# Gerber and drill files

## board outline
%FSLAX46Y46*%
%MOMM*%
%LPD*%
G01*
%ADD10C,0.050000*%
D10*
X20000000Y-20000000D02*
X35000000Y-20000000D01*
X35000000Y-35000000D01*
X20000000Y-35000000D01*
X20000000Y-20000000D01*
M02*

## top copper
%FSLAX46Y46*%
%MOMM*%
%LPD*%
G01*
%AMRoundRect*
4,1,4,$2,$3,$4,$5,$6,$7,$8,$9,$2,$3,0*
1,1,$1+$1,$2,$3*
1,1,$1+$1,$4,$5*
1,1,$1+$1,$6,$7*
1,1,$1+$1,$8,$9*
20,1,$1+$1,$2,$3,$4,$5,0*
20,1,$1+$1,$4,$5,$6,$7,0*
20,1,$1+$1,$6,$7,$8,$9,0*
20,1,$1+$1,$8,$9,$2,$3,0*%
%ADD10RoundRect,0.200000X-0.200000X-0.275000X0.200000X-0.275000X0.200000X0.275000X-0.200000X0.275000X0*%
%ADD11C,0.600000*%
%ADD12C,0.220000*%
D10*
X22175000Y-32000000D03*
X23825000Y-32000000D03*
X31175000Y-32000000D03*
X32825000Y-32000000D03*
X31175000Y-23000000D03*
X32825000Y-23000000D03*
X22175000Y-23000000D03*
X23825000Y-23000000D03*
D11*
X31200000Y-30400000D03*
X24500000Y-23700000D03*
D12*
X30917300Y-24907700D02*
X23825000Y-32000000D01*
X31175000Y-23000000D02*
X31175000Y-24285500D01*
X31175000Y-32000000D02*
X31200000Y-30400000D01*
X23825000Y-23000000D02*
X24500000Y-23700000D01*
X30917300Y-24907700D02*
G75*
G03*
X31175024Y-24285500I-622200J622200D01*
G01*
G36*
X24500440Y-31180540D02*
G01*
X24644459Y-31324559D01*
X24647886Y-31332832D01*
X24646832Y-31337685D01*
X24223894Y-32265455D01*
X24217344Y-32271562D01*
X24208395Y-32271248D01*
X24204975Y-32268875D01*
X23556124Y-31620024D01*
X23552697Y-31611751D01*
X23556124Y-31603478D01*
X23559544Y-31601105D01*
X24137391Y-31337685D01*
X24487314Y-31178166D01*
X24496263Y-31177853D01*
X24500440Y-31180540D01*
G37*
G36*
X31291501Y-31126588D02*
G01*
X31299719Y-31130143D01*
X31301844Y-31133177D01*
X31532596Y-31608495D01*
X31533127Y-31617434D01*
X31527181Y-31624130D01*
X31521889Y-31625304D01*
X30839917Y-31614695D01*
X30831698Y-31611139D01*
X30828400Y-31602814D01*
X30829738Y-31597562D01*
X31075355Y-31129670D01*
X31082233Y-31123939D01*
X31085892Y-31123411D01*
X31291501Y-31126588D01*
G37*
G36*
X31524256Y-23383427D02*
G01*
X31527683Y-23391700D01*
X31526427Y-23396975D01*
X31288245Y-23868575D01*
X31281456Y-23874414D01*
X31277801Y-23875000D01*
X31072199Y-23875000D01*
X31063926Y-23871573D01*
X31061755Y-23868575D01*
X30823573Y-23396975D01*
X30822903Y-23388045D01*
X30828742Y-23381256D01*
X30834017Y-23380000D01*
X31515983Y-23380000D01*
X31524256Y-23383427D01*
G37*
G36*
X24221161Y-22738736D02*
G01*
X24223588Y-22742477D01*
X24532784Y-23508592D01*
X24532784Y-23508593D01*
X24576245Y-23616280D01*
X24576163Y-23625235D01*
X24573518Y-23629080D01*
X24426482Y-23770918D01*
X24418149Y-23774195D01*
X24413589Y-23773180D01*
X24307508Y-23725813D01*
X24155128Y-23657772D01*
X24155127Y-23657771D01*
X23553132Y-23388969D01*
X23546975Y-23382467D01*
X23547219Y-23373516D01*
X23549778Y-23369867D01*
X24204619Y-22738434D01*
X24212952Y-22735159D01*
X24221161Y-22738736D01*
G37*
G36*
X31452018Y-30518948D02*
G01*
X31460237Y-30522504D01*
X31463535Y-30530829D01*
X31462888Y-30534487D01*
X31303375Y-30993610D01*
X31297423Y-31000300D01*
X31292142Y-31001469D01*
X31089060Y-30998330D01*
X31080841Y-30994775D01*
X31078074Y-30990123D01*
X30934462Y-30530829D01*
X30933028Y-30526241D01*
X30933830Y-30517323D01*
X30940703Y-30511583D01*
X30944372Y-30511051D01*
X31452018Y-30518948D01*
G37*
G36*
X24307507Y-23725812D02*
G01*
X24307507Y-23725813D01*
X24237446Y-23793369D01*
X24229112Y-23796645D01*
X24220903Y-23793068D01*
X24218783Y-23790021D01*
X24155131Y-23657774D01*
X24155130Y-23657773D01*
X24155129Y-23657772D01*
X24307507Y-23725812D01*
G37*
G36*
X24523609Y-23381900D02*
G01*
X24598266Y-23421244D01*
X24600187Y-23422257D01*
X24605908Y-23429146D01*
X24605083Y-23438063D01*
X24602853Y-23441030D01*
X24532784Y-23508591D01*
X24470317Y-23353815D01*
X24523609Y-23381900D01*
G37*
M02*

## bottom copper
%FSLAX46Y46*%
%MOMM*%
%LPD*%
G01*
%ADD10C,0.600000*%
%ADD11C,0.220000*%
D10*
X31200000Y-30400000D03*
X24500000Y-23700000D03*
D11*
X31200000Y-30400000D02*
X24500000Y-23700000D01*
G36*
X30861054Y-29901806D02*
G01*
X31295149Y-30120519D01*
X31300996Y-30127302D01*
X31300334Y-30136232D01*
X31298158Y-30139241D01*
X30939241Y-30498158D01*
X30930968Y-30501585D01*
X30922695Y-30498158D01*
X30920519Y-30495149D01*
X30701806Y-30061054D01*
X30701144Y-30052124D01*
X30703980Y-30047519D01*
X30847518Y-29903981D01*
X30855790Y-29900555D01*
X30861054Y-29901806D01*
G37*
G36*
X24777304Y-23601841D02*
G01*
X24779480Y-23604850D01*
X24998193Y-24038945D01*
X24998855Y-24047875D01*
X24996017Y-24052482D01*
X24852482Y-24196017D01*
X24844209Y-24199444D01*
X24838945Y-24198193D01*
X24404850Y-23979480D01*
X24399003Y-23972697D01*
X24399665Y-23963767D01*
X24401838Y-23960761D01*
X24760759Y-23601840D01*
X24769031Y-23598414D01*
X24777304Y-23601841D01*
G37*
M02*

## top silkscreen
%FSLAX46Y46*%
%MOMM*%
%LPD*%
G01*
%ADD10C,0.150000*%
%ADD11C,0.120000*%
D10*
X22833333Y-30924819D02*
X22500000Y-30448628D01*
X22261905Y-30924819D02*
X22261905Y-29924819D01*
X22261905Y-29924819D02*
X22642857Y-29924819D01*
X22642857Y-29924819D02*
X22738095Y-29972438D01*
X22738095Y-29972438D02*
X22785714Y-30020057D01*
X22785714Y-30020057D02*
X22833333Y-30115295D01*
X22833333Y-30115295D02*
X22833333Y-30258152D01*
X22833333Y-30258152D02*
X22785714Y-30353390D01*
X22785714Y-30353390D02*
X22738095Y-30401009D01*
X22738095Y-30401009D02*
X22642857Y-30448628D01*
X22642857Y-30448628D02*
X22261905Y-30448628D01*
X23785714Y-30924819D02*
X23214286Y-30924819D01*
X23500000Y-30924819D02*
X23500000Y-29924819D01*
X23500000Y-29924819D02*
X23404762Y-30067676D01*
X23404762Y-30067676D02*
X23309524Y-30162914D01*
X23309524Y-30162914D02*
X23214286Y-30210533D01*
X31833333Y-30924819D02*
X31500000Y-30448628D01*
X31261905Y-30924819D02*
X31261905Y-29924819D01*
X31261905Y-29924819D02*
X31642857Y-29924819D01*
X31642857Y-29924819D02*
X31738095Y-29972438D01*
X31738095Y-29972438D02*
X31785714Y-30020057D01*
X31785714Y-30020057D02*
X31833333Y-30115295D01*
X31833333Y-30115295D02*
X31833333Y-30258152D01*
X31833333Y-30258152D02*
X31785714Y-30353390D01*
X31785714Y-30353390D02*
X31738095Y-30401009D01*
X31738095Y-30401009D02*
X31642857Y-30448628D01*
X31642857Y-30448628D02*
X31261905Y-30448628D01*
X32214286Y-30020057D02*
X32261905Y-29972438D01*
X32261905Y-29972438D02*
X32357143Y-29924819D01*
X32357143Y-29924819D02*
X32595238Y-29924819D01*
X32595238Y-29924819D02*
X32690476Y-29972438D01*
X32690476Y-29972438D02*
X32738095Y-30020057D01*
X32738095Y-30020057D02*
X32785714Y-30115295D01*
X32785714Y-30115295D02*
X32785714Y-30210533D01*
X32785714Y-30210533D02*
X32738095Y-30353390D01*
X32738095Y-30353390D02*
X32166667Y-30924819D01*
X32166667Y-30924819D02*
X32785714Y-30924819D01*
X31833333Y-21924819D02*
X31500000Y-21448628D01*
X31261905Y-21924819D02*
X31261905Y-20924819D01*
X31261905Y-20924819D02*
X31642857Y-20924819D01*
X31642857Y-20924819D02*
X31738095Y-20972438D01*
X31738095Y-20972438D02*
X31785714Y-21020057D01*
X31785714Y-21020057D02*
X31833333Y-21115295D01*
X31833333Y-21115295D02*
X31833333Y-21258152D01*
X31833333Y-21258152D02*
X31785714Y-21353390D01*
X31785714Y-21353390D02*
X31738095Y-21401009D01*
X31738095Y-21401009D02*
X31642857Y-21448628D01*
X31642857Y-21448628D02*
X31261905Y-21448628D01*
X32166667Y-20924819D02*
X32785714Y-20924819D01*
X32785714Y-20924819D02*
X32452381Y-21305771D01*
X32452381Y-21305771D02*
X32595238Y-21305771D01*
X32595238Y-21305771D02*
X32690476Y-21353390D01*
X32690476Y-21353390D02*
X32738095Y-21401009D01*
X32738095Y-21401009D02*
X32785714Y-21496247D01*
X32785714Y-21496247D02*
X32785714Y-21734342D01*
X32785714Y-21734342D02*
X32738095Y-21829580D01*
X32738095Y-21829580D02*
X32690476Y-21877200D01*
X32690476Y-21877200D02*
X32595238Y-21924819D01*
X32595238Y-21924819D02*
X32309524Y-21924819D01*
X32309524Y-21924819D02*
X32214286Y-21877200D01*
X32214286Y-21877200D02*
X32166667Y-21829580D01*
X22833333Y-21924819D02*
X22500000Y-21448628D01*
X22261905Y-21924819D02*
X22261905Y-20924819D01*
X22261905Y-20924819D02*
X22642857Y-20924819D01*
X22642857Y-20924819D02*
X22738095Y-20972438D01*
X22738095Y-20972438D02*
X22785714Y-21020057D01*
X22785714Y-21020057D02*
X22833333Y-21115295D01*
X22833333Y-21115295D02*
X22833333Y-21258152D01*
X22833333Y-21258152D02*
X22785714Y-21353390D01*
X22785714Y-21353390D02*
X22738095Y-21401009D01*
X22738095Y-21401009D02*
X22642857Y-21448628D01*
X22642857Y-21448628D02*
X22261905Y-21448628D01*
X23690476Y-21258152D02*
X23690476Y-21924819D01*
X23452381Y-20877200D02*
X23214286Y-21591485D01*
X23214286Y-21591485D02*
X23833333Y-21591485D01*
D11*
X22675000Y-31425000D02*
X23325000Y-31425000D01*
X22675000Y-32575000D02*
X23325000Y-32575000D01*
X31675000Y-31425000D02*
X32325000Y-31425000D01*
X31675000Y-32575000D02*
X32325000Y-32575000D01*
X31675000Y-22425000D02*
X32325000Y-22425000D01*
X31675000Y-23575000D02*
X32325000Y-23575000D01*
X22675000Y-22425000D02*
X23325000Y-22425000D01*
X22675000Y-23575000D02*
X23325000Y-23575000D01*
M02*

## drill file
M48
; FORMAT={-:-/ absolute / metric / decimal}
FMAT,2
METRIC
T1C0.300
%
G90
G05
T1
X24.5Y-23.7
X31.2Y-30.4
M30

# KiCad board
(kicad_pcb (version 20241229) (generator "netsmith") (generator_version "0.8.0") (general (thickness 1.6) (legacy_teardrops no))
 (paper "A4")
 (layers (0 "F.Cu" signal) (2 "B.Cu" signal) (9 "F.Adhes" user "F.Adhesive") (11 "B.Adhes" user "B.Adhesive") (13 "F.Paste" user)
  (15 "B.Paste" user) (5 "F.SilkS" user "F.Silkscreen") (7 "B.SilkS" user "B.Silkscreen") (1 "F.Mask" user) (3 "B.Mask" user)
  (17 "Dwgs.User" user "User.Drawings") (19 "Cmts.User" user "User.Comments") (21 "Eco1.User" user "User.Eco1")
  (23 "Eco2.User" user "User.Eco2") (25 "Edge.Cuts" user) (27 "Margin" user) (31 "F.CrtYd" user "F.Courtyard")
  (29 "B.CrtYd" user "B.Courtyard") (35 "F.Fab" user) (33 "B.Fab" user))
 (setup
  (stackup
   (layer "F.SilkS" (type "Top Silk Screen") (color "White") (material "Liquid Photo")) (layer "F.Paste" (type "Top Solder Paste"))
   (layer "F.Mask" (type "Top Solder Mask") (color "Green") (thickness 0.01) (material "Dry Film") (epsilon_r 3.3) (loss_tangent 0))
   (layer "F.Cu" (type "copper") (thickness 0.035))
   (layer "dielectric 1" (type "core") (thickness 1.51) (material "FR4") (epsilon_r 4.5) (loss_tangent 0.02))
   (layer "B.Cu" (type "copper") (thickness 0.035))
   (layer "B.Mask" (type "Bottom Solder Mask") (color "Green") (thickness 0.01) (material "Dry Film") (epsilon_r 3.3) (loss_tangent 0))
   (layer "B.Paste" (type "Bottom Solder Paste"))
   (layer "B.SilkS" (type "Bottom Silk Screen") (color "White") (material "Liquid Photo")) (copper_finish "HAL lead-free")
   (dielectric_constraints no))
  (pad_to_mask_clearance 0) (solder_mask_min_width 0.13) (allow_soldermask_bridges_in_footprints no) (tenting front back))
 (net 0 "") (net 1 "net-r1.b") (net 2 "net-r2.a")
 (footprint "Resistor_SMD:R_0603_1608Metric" (layer "F.Cu") (at 23 32)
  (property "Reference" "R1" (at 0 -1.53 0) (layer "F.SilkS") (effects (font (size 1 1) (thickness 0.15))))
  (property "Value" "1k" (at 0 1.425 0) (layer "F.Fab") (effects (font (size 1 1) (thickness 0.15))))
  (pad "1" smd roundrect (at -0.825 0) (size 0.8 0.95) (layers "F.Cu" "F.Mask" "F.Paste") (roundrect_rratio 0.25))
  (pad "2" smd roundrect (at 0.825 0) (size 0.8 0.95) (layers "F.Cu" "F.Mask" "F.Paste") (roundrect_rratio 0.25) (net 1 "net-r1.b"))
  (fp_line (start -0.325 -0.575) (end 0.325 -0.575) (stroke (width 0.12) (type solid)) (layer "F.SilkS"))
  (fp_line (start -0.325 0.575) (end 0.325 0.575) (stroke (width 0.12) (type solid)) (layer "F.SilkS")))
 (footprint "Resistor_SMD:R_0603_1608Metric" (layer "F.Cu") (at 32 32)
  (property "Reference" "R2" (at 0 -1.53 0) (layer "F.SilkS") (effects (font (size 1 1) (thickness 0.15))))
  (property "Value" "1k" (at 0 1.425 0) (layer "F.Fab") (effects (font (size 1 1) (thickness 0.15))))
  (pad "1" smd roundrect (at -0.825 0) (size 0.8 0.95) (layers "F.Cu" "F.Mask" "F.Paste") (roundrect_rratio 0.25) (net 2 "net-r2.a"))
  (pad "2" smd roundrect (at 0.825 0) (size 0.8 0.95) (layers "F.Cu" "F.Mask" "F.Paste") (roundrect_rratio 0.25))
  (fp_line (start -0.325 -0.575) (end 0.325 -0.575) (stroke (width 0.12) (type solid)) (layer "F.SilkS"))
  (fp_line (start -0.325 0.575) (end 0.325 0.575) (stroke (width 0.12) (type solid)) (layer "F.SilkS")))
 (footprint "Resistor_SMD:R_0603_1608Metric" (layer "F.Cu") (at 32 23)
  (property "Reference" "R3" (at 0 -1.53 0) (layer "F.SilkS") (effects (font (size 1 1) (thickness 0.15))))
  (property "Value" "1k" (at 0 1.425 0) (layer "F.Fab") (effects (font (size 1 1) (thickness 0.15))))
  (pad "1" smd roundrect (at -0.825 0) (size 0.8 0.95) (layers "F.Cu" "F.Mask" "F.Paste") (roundrect_rratio 0.25) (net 1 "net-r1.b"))
  (pad "2" smd roundrect (at 0.825 0) (size 0.8 0.95) (layers "F.Cu" "F.Mask" "F.Paste") (roundrect_rratio 0.25))
  (fp_line (start -0.325 -0.575) (end 0.325 -0.575) (stroke (width 0.12) (type solid)) (layer "F.SilkS"))
  (fp_line (start -0.325 0.575) (end 0.325 0.575) (stroke (width 0.12) (type solid)) (layer "F.SilkS")))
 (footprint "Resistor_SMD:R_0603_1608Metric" (layer "F.Cu") (at 23 23)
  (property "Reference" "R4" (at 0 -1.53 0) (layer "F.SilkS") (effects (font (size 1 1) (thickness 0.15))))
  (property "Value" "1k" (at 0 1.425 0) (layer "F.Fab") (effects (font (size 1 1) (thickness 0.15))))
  (pad "1" smd roundrect (at -0.825 0) (size 0.8 0.95) (layers "F.Cu" "F.Mask" "F.Paste") (roundrect_rratio 0.25))
  (pad "2" smd roundrect (at 0.825 0) (size 0.8 0.95) (layers "F.Cu" "F.Mask" "F.Paste") (roundrect_rratio 0.25) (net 2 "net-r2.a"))
  (fp_line (start -0.325 -0.575) (end 0.325 -0.575) (stroke (width 0.12) (type solid)) (layer "F.SilkS"))
  (fp_line (start -0.325 0.575) (end 0.325 0.575) (stroke (width 0.12) (type solid)) (layer "F.SilkS")))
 (segment (start 30.9173 24.9077) (end 23.825 32) (width 0.22) (layer "F.Cu") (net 1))
 (segment (start 31.175 23) (end 31.175 24.2855) (width 0.22) (layer "F.Cu") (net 1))
 (segment (start 31.175 32) (end 31.2 30.4) (width 0.22) (layer "F.Cu") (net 2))
 (segment (start 31.2 30.4) (end 24.5 23.7) (width 0.22) (layer "B.Cu") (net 2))
 (segment (start 23.825 23) (end 24.5 23.7) (width 0.22) (layer "F.Cu") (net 2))
 (arc (start 30.9173 24.9077) (mid 31.108 24.6223) (end 31.175 24.2855) (width 0.22) (layer "F.Cu") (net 1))
 (via (at 31.2 30.4) (size 0.6) (drill 0.3) (layers "F.Cu" "B.Cu") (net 2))
 (via (at 24.5 23.7) (size 0.6) (drill 0.3) (layers "F.Cu" "B.Cu") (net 2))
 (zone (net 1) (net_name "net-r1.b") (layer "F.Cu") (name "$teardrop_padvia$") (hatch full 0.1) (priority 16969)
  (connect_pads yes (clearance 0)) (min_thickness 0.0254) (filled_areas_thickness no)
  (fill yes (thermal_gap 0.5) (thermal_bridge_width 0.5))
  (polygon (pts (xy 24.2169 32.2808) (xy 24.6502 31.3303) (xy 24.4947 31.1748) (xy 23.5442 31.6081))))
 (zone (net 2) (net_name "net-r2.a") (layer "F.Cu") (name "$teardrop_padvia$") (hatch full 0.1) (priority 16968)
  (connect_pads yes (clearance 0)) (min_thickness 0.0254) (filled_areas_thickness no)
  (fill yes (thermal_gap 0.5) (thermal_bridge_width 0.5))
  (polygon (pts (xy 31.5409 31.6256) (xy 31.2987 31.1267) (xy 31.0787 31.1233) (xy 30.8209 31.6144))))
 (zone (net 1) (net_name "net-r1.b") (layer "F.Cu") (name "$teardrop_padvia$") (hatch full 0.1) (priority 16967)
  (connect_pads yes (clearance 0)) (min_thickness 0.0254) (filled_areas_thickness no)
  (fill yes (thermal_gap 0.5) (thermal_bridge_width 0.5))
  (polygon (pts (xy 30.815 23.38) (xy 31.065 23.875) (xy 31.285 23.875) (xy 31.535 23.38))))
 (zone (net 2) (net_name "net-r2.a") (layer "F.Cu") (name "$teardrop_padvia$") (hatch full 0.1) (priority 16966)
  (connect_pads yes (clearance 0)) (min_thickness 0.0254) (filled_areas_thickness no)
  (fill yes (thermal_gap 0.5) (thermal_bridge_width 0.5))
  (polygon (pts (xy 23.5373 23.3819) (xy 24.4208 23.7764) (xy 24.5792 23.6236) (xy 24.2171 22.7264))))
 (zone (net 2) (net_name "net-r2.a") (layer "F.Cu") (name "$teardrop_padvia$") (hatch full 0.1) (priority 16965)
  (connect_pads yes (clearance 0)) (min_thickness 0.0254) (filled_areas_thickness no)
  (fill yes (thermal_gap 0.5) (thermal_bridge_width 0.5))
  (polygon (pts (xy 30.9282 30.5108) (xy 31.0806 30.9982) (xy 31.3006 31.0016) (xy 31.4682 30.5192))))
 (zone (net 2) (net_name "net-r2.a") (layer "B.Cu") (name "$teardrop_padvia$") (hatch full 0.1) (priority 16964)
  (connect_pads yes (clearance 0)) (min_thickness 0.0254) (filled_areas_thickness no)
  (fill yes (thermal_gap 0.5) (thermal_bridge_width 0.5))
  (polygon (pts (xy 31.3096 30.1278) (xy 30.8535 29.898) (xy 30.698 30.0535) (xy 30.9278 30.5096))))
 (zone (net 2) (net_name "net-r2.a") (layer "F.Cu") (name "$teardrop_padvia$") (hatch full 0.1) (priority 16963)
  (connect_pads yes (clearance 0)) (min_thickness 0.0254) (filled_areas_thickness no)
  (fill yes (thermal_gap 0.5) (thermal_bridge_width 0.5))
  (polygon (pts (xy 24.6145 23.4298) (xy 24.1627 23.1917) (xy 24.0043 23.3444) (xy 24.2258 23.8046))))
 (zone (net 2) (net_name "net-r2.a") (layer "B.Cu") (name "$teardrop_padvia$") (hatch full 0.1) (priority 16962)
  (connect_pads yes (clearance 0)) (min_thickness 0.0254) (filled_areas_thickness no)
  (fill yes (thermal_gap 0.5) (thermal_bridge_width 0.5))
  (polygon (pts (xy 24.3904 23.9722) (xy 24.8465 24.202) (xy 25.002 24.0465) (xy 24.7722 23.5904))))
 (gr_rect (start 20 20) (end 35 35) (stroke (width 0.05) (type default)) (fill no) (layer "Edge.Cuts")))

